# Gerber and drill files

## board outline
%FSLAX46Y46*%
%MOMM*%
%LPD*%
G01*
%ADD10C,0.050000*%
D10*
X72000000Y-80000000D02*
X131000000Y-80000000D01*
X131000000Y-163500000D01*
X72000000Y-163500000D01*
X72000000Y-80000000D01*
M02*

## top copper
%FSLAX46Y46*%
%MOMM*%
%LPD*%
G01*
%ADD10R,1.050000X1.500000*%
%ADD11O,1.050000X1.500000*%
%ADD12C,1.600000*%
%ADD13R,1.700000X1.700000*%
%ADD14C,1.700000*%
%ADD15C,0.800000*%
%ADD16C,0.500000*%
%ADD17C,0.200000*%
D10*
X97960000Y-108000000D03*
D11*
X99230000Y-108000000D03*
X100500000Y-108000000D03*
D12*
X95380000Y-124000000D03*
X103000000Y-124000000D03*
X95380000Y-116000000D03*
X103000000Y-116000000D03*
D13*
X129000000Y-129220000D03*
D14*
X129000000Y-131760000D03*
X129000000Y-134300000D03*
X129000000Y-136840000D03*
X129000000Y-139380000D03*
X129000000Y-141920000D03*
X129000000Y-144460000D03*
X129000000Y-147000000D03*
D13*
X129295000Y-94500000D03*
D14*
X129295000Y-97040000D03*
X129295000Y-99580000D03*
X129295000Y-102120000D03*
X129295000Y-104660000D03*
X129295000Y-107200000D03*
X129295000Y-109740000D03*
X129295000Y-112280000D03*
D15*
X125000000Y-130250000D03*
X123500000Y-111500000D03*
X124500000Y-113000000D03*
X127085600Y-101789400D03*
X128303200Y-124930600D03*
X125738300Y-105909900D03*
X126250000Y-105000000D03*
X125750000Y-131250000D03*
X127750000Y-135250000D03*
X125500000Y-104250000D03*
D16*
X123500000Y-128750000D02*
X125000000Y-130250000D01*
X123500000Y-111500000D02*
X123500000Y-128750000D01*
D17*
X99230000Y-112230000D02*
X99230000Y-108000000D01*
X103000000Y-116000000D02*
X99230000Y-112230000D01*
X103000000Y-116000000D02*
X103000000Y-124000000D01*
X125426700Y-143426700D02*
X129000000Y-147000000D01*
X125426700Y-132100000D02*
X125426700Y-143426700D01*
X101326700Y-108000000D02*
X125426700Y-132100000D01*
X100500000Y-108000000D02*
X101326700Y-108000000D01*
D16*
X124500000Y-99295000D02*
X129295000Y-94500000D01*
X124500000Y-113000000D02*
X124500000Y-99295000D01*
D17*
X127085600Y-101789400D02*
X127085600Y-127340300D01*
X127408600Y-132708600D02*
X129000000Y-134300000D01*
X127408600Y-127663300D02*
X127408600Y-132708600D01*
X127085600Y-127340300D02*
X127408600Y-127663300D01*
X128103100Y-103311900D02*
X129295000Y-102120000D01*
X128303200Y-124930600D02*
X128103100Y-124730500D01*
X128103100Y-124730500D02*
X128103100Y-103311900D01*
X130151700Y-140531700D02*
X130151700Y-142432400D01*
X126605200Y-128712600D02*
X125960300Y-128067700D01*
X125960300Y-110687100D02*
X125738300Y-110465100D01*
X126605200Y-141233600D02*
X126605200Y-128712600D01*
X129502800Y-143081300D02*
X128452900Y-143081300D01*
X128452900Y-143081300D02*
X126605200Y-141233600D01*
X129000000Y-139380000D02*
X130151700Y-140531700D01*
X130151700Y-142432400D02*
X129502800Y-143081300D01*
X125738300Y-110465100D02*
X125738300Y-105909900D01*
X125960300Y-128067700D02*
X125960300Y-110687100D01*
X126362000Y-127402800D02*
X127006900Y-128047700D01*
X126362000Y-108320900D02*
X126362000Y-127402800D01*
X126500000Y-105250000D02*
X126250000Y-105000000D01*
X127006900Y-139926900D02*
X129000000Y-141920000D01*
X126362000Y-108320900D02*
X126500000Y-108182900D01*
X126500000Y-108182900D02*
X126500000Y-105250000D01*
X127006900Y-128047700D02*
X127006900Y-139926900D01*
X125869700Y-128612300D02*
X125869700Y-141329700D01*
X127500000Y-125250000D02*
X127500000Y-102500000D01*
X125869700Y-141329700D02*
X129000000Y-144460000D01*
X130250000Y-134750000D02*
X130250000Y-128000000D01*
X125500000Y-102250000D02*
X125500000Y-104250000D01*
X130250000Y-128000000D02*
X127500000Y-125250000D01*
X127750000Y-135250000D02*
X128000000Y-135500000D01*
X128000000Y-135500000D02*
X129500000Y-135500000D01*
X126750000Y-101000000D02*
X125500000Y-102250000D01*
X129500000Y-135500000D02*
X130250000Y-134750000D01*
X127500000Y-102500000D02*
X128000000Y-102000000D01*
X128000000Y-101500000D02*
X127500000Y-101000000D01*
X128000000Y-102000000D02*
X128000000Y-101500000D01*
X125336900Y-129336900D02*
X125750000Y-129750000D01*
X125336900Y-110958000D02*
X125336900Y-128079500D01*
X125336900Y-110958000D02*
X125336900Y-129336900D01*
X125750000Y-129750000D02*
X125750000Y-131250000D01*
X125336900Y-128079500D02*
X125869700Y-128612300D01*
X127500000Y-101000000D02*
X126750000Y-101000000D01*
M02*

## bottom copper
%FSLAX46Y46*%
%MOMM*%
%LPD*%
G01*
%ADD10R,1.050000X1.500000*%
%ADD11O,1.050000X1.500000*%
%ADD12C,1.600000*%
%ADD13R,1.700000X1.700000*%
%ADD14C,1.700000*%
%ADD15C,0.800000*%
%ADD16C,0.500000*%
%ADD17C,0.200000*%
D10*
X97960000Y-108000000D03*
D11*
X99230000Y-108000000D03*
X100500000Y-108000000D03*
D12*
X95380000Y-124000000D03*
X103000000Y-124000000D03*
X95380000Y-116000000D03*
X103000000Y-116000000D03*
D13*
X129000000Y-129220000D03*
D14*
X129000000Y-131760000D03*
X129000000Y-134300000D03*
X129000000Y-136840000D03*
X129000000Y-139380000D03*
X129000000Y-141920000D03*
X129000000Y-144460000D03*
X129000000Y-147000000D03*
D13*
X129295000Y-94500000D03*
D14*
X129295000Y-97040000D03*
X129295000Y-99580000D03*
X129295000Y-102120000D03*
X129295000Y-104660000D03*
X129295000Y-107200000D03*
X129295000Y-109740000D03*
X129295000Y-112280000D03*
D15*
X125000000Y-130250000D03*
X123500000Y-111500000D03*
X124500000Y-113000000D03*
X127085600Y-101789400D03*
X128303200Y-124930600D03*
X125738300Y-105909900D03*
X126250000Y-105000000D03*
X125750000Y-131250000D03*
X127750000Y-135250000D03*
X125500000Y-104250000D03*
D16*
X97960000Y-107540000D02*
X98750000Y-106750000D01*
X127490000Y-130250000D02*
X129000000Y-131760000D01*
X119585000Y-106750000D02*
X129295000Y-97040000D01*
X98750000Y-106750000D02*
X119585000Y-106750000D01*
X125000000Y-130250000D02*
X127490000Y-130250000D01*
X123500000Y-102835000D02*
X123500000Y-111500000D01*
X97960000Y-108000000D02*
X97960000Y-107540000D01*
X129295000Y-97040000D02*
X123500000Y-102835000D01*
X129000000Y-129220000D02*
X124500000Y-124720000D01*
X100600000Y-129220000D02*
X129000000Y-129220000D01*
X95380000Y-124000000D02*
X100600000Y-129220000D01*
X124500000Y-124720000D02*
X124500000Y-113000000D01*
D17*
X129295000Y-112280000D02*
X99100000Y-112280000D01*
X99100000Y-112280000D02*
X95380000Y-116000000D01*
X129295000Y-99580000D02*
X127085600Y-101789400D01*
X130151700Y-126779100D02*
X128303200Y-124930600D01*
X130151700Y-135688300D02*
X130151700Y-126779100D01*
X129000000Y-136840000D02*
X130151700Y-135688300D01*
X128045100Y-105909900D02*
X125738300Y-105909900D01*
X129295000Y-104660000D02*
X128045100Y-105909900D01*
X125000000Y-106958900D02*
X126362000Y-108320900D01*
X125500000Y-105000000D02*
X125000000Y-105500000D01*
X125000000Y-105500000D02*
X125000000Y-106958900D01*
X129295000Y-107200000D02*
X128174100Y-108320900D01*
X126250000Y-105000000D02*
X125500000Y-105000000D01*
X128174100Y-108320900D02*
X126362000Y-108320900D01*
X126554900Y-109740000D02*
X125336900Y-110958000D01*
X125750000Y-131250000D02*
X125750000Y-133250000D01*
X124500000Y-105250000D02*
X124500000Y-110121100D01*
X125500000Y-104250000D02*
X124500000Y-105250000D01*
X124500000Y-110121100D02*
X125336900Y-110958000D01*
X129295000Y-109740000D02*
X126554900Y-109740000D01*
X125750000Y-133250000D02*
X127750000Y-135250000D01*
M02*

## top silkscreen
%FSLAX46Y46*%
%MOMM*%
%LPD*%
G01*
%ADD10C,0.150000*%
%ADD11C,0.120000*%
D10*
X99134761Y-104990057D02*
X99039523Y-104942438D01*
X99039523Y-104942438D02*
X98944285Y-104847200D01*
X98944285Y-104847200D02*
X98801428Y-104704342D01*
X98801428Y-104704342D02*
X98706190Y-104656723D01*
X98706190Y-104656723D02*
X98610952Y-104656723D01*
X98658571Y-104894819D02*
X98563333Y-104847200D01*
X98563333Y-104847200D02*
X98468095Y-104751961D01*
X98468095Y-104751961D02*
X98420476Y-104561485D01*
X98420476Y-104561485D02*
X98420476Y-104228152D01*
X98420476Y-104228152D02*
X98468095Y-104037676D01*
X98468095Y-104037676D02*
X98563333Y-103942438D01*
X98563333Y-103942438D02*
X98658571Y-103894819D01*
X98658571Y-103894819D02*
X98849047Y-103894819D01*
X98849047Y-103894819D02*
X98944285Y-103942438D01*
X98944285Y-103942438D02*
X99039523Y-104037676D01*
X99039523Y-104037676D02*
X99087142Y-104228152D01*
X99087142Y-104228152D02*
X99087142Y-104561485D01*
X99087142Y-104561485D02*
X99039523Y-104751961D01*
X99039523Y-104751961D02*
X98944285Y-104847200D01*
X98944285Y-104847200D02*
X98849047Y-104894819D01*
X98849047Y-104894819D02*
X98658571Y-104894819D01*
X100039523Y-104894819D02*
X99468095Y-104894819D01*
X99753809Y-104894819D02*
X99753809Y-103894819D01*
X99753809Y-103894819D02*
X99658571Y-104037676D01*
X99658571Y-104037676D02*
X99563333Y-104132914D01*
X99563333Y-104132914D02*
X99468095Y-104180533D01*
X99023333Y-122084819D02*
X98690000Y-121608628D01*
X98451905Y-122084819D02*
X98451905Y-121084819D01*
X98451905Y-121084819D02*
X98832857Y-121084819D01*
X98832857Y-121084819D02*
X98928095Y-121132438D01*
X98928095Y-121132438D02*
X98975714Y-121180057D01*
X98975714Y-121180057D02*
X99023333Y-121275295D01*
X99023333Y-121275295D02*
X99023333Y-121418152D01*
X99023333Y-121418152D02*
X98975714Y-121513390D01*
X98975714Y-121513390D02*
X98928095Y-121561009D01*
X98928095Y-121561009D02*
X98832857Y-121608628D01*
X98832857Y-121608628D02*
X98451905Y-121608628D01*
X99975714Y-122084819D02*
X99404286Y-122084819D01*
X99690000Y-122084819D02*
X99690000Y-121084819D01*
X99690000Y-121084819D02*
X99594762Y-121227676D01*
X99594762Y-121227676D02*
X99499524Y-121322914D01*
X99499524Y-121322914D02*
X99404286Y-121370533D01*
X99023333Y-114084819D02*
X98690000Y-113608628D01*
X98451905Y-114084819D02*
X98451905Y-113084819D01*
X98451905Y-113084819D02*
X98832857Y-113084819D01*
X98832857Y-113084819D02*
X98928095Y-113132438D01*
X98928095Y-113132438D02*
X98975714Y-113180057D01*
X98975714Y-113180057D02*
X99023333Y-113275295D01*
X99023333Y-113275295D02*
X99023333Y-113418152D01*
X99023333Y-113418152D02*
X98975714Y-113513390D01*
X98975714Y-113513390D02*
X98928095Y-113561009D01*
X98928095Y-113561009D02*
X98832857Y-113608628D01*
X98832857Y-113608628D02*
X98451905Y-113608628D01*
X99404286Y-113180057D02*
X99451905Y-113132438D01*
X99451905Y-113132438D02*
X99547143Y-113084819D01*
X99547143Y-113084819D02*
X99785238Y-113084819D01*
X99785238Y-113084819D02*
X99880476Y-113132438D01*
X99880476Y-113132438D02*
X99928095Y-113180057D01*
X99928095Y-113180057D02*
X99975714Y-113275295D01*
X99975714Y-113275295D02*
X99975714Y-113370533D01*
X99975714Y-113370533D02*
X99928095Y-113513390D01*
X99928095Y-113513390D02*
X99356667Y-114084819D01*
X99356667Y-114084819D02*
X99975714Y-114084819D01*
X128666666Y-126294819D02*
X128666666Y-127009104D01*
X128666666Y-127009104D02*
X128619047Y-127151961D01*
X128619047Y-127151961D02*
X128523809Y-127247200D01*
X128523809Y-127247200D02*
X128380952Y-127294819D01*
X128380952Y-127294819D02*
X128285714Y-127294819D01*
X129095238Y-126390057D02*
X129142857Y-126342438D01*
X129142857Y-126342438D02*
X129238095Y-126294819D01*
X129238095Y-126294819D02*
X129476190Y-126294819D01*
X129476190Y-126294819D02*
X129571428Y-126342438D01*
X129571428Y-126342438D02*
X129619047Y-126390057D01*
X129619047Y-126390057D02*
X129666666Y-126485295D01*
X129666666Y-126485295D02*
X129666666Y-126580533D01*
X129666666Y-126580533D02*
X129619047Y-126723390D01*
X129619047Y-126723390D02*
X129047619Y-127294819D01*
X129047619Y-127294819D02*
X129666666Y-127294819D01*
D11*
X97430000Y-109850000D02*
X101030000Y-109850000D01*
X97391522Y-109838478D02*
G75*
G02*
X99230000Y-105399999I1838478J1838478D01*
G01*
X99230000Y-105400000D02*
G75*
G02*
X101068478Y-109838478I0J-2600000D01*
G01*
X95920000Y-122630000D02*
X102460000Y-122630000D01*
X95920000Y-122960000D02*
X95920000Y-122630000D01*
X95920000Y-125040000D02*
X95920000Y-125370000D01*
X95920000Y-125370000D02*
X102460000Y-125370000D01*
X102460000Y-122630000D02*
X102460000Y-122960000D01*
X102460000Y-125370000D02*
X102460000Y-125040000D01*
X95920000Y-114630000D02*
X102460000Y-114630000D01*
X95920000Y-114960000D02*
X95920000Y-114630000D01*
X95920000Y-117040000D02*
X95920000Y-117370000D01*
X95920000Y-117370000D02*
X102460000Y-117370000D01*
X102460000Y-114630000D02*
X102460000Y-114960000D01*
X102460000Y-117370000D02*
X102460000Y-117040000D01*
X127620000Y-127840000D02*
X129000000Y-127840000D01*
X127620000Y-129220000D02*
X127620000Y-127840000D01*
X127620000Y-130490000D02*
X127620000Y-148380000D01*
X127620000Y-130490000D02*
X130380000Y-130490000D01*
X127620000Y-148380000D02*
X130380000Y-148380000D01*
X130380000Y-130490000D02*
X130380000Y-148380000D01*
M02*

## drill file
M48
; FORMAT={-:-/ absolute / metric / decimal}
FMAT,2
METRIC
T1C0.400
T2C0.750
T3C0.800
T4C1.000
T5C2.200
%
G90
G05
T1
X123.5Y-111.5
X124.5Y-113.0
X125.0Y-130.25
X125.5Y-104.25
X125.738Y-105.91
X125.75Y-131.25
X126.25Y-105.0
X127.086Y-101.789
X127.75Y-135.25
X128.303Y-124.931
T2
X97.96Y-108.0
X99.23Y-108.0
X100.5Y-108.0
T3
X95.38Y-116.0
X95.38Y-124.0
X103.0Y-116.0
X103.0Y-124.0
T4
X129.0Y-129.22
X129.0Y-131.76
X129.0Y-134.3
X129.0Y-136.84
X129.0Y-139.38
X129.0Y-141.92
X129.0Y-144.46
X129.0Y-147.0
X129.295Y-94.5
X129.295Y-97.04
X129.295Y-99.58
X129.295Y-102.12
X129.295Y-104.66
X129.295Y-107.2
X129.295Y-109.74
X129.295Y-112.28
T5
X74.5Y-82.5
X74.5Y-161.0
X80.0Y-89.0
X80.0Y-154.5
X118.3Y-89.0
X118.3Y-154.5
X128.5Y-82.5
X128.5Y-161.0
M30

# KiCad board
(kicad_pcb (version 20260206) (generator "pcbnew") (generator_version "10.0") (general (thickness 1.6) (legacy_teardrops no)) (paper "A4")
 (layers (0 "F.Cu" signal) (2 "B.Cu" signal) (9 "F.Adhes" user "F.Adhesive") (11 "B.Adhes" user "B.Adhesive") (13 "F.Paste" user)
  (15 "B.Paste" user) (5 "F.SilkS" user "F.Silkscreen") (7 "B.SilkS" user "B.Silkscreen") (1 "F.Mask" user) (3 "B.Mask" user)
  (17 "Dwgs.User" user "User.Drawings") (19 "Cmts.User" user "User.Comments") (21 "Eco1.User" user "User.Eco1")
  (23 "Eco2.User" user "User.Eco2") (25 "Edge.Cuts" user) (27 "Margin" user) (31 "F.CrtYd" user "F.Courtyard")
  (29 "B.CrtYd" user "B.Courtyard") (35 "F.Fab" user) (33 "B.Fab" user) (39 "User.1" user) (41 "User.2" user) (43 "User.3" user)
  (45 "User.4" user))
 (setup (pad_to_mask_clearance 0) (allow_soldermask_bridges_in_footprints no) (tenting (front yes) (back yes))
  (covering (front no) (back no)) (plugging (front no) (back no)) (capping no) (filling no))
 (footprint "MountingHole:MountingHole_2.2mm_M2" (layer "F.Cu") (at 118.3 89)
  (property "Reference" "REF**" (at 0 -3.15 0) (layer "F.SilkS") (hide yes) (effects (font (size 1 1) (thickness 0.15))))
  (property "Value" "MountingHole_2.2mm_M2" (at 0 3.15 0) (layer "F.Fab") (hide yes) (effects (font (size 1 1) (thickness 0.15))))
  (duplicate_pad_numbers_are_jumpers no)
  (pad "" np_thru_hole circle (at 0 0) (size 2.2 2.2) (drill 2.2) (layers "*.Cu" "*.Mask")))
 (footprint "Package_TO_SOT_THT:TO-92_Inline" (layer "F.Cu") (at 97.96 108)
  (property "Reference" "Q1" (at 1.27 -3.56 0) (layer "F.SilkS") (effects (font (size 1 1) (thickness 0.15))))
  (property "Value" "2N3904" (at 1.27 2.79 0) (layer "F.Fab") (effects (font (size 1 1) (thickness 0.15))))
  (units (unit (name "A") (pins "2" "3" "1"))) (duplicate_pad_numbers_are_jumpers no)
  (fp_line (start -0.53 1.85) (end 3.07 1.85) (stroke (width 0.12) (type solid)) (layer "F.SilkS"))
  (fp_arc (start -0.568478 1.838478) (mid -1.132087 -0.994977) (end 1.27 -2.6) (stroke (width 0.12) (type solid)) (layer "F.SilkS"))
  (fp_arc (start 1.27 -2.6) (mid 3.672087 -0.994977) (end 3.108478 1.838478) (stroke (width 0.12) (type solid)) (layer "F.SilkS"))
  (pad "1" thru_hole rect (at 0 0) (size 1.05 1.5) (drill 0.75) (layers "*.Cu" "*.Mask") (remove_unused_layers no) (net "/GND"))
  (pad "2" thru_hole oval (at 1.27 0) (size 1.05 1.5) (drill 0.75) (layers "*.Cu" "*.Mask") (remove_unused_layers no) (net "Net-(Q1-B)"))
  (pad "3" thru_hole oval (at 2.54 0) (size 1.05 1.5) (drill 0.75) (layers "*.Cu" "*.Mask") (remove_unused_layers no) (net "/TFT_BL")))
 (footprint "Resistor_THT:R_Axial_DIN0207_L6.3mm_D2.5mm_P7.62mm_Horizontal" (layer "F.Cu") (at 95.38 124)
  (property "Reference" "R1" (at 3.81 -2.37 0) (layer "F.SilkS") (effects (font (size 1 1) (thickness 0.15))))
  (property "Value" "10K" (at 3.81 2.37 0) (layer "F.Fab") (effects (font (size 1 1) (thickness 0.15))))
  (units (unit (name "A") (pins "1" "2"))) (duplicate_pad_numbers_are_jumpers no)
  (fp_line (start 0.54 -1.37) (end 7.08 -1.37) (stroke (width 0.12) (type solid)) (layer "F.SilkS"))
  (fp_line (start 0.54 -1.04) (end 0.54 -1.37) (stroke (width 0.12) (type solid)) (layer "F.SilkS"))
  (fp_line (start 0.54 1.04) (end 0.54 1.37) (stroke (width 0.12) (type solid)) (layer "F.SilkS"))
  (fp_line (start 0.54 1.37) (end 7.08 1.37) (stroke (width 0.12) (type solid)) (layer "F.SilkS"))
  (fp_line (start 7.08 -1.37) (end 7.08 -1.04) (stroke (width 0.12) (type solid)) (layer "F.SilkS"))
  (fp_line (start 7.08 1.37) (end 7.08 1.04) (stroke (width 0.12) (type solid)) (layer "F.SilkS"))
  (pad "1" thru_hole circle (at 0 0) (size 1.6 1.6) (drill 0.8) (layers "*.Cu" "*.Mask") (remove_unused_layers no) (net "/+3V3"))
  (pad "2" thru_hole circle (at 7.62 0) (size 1.6 1.6) (drill 0.8) (layers "*.Cu" "*.Mask") (remove_unused_layers no) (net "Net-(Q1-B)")))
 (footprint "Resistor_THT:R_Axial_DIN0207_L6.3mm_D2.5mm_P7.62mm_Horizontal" (layer "F.Cu") (at 95.38 116)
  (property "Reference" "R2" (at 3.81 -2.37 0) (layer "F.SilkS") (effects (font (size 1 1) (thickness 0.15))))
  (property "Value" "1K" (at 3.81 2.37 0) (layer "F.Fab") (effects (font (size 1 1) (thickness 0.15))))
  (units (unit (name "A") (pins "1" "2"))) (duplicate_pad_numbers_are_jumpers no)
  (fp_line (start 0.54 -1.37) (end 7.08 -1.37) (stroke (width 0.12) (type solid)) (layer "F.SilkS"))
  (fp_line (start 0.54 -1.04) (end 0.54 -1.37) (stroke (width 0.12) (type solid)) (layer "F.SilkS"))
  (fp_line (start 0.54 1.04) (end 0.54 1.37) (stroke (width 0.12) (type solid)) (layer "F.SilkS"))
  (fp_line (start 0.54 1.37) (end 7.08 1.37) (stroke (width 0.12) (type solid)) (layer "F.SilkS"))
  (fp_line (start 7.08 -1.37) (end 7.08 -1.04) (stroke (width 0.12) (type solid)) (layer "F.SilkS"))
  (fp_line (start 7.08 1.37) (end 7.08 1.04) (stroke (width 0.12) (type solid)) (layer "F.SilkS"))
  (pad "1" thru_hole circle (at 0 0) (size 1.6 1.6) (drill 0.8) (layers "*.Cu" "*.Mask") (remove_unused_layers no) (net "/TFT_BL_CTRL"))
  (pad "2" thru_hole circle (at 7.62 0) (size 1.6 1.6) (drill 0.8) (layers "*.Cu" "*.Mask") (remove_unused_layers no) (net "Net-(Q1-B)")))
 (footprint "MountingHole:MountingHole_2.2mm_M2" (layer "F.Cu") (at 80 154.5)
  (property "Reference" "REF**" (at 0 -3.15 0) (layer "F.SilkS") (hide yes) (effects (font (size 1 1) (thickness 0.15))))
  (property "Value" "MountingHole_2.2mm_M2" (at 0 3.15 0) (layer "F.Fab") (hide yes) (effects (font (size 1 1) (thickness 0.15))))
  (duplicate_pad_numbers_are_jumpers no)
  (pad "" np_thru_hole circle (at 0 0) (size 2.2 2.2) (drill 2.2) (layers "*.Cu" "*.Mask")))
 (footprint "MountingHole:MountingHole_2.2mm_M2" (layer "F.Cu") (at 128.5 161)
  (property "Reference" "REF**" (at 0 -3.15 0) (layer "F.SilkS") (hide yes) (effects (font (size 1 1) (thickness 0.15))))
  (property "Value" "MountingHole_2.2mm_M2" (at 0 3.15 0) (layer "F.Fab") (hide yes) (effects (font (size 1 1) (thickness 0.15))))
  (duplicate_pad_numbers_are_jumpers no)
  (pad "" np_thru_hole circle (at 0 0) (size 2.2 2.2) (drill 2.2) (layers "*.Cu" "*.Mask")))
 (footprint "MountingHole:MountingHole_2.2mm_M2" (layer "F.Cu") (at 128.5 82.5)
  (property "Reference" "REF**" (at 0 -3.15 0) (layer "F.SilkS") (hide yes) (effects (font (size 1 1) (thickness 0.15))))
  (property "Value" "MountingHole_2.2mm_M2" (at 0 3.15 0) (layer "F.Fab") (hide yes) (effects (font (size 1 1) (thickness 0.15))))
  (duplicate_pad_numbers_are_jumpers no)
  (pad "" np_thru_hole circle (at 0 0) (size 2.2 2.2) (drill 2.2) (layers "*.Cu" "*.Mask")))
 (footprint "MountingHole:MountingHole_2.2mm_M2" (layer "F.Cu") (at 80 89)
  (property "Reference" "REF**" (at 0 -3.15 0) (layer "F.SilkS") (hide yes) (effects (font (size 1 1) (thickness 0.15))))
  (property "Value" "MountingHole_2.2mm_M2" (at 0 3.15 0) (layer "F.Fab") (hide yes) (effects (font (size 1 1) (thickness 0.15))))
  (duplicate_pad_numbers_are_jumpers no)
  (pad "" np_thru_hole circle (at 0 0) (size 2.2 2.2) (drill 2.2) (layers "*.Cu" "*.Mask")))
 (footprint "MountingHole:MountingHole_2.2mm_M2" (layer "F.Cu") (at 118.3 154.5)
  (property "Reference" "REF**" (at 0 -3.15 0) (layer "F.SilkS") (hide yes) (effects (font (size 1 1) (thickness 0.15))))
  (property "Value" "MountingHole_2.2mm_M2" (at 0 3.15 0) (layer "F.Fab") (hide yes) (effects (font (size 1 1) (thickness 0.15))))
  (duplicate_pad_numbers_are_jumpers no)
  (pad "" np_thru_hole circle (at 0 0) (size 2.2 2.2) (drill 2.2) (layers "*.Cu" "*.Mask")))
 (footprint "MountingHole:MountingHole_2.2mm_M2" (layer "F.Cu") (at 74.5 82.5)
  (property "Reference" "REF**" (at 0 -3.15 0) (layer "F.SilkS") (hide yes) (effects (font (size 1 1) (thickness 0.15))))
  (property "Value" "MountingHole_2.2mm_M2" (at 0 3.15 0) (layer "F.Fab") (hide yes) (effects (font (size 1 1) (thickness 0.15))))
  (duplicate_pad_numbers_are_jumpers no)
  (pad "" np_thru_hole circle (at 0 0) (size 2.2 2.2) (drill 2.2) (layers "*.Cu" "*.Mask")))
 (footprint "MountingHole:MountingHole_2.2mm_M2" (layer "F.Cu") (at 74.5 161)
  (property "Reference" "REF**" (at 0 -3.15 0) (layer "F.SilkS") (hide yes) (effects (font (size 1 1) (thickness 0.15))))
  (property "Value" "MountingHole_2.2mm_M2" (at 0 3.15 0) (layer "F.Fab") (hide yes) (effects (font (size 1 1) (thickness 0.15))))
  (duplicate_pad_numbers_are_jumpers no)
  (pad "" np_thru_hole circle (at 0 0) (size 2.2 2.2) (drill 2.2) (layers "*.Cu" "*.Mask")))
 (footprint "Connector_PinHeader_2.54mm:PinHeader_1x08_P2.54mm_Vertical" (layer "F.Cu") (at 129 129.22)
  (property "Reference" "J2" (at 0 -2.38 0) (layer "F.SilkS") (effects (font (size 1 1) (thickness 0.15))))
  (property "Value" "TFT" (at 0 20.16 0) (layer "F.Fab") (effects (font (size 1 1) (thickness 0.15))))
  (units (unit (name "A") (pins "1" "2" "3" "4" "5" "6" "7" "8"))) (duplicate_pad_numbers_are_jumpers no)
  (fp_line (start -1.38 -1.38) (end 0 -1.38) (stroke (width 0.12) (type solid)) (layer "F.SilkS"))
  (fp_line (start -1.38 0) (end -1.38 -1.38) (stroke (width 0.12) (type solid)) (layer "F.SilkS"))
  (fp_line (start -1.38 1.27) (end -1.38 19.16) (stroke (width 0.12) (type solid)) (layer "F.SilkS"))
  (fp_line (start -1.38 1.27) (end 1.38 1.27) (stroke (width 0.12) (type solid)) (layer "F.SilkS"))
  (fp_line (start -1.38 19.16) (end 1.38 19.16) (stroke (width 0.12) (type solid)) (layer "F.SilkS"))
  (fp_line (start 1.38 1.27) (end 1.38 19.16) (stroke (width 0.12) (type solid)) (layer "F.SilkS"))
  (pad "1" thru_hole rect (at 0 0) (size 1.7 1.7) (drill 1) (layers "*.Cu" "*.Mask") (remove_unused_layers no) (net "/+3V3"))
  (pad "2" thru_hole circle (at 0 2.54) (size 1.7 1.7) (drill 1) (layers "*.Cu" "*.Mask") (remove_unused_layers no) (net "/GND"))
  (pad "3" thru_hole circle (at 0 5.08) (size 1.7 1.7) (drill 1) (layers "*.Cu" "*.Mask") (remove_unused_layers no) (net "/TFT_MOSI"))
  (pad "4" thru_hole circle (at 0 7.62) (size 1.7 1.7) (drill 1) (layers "*.Cu" "*.Mask") (remove_unused_layers no) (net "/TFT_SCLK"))
  (pad "5" thru_hole circle (at 0 10.16) (size 1.7 1.7) (drill 1) (layers "*.Cu" "*.Mask") (remove_unused_layers no) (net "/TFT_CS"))
  (pad "6" thru_hole circle (at 0 12.7) (size 1.7 1.7) (drill 1) (layers "*.Cu" "*.Mask") (remove_unused_layers no) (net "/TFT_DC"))
  (pad "7" thru_hole circle (at 0 15.24) (size 1.7 1.7) (drill 1) (layers "*.Cu" "*.Mask") (remove_unused_layers no) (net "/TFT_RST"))
  (pad "8" thru_hole circle (at 0 17.78) (size 1.7 1.7) (drill 1) (layers "*.Cu" "*.Mask") (remove_unused_layers no) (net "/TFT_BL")))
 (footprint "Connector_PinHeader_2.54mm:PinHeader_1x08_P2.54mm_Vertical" (layer "B.Cu") (at 129.295 94.5 180)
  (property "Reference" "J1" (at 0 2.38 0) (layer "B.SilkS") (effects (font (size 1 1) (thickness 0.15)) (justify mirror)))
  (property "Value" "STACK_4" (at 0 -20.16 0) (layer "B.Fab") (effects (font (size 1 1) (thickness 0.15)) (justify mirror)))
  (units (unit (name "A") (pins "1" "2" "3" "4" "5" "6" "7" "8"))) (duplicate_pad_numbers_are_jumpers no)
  (pad "1" thru_hole rect (at 0 0 180) (size 1.7 1.7) (drill 1) (layers "*.Cu" "*.Mask") (remove_unused_layers no) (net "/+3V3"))
  (pad "2" thru_hole circle (at 0 -2.54 180) (size 1.7 1.7) (drill 1) (layers "*.Cu" "*.Mask") (remove_unused_layers no) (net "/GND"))
  (pad "3" thru_hole circle (at 0 -5.08 180) (size 1.7 1.7) (drill 1) (layers "*.Cu" "*.Mask") (remove_unused_layers no) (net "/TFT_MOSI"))
  (pad "4" thru_hole circle (at 0 -7.62 180) (size 1.7 1.7) (drill 1) (layers "*.Cu" "*.Mask") (remove_unused_layers no) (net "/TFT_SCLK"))
  (pad "5" thru_hole circle (at 0 -10.16 180) (size 1.7 1.7) (drill 1) (layers "*.Cu" "*.Mask") (remove_unused_layers no) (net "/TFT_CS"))
  (pad "6" thru_hole circle (at 0 -12.7 180) (size 1.7 1.7) (drill 1) (layers "*.Cu" "*.Mask") (remove_unused_layers no) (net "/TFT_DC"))
  (pad "7" thru_hole circle (at 0 -15.24 180) (size 1.7 1.7) (drill 1) (layers "*.Cu" "*.Mask") (remove_unused_layers no) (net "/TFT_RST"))
  (pad "8" thru_hole circle (at 0 -17.78 180) (size 1.7 1.7) (drill 1) (layers "*.Cu" "*.Mask") (remove_unused_layers no)
   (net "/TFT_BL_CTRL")))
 (gr_rect (start 72 80) (end 131 163.5) (stroke (width 0.05) (type default)) (fill no) (layer "Edge.Cuts"))
 (segment (start 123.5 128.75) (end 125 130.25) (width 0.5) (layer "F.Cu") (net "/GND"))
 (segment (start 123.5 111.5) (end 123.5 128.75) (width 0.5) (layer "F.Cu") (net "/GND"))
 (via (at 125 130.25) (size 0.8) (drill 0.4) (layers "F.Cu" "B.Cu") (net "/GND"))
 (via (at 123.5 111.5) (size 0.8) (drill 0.4) (layers "F.Cu" "B.Cu") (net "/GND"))
 (segment (start 97.96 107.54) (end 98.75 106.75) (width 0.5) (layer "B.Cu") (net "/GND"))
 (segment (start 127.49 130.25) (end 129 131.76) (width 0.5) (layer "B.Cu") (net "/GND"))
 (segment (start 119.585 106.75) (end 129.295 97.04) (width 0.5) (layer "B.Cu") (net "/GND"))
 (segment (start 98.75 106.75) (end 119.585 106.75) (width 0.5) (layer "B.Cu") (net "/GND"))
 (segment (start 125 130.25) (end 127.49 130.25) (width 0.5) (layer "B.Cu") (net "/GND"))
 (segment (start 123.5 102.835) (end 123.5 111.5) (width 0.5) (layer "B.Cu") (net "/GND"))
 (segment (start 97.96 108) (end 97.96 107.54) (width 0.5) (layer "B.Cu") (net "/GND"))
 (segment (start 129.295 97.04) (end 123.5 102.835) (width 0.5) (layer "B.Cu") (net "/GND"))
 (segment (start 99.23 112.23) (end 99.23 108) (width 0.2) (layer "F.Cu") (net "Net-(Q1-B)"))
 (segment (start 103 116) (end 99.23 112.23) (width 0.2) (layer "F.Cu") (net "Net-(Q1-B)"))
 (segment (start 103 116) (end 103 124) (width 0.2) (layer "F.Cu") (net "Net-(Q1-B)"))
 (segment (start 125.4267 143.4267) (end 129 147) (width 0.2) (layer "F.Cu") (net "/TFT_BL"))
 (segment (start 125.4267 132.1) (end 125.4267 143.4267) (width 0.2) (layer "F.Cu") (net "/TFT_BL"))
 (segment (start 101.3267 108) (end 125.4267 132.1) (width 0.2) (layer "F.Cu") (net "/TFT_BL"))
 (segment (start 100.5 108) (end 101.3267 108) (width 0.2) (layer "F.Cu") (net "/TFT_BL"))
 (segment (start 124.5 99.295) (end 129.295 94.5) (width 0.5) (layer "F.Cu") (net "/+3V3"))
 (segment (start 124.5 113) (end 124.5 99.295) (width 0.5) (layer "F.Cu") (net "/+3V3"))
 (via (at 124.5 113) (size 0.8) (drill 0.4) (layers "F.Cu" "B.Cu") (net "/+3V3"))
 (segment (start 129 129.22) (end 124.5 124.72) (width 0.5) (layer "B.Cu") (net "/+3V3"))
 (segment (start 100.6 129.22) (end 129 129.22) (width 0.5) (layer "B.Cu") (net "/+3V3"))
 (segment (start 95.38 124) (end 100.6 129.22) (width 0.5) (layer "B.Cu") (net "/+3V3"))
 (segment (start 124.5 124.72) (end 124.5 113) (width 0.5) (layer "B.Cu") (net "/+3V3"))
 (segment (start 129.295 112.28) (end 99.1 112.28) (width 0.2) (layer "B.Cu") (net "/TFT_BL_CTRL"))
 (segment (start 99.1 112.28) (end 95.38 116) (width 0.2) (layer "B.Cu") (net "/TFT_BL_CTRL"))
 (segment (start 127.0856 101.7894) (end 127.0856 127.3403) (width 0.2) (layer "F.Cu") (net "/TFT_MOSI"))
 (segment (start 127.4086 132.7086) (end 129 134.3) (width 0.2) (layer "F.Cu") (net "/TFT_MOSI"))
 (segment (start 127.4086 127.6633) (end 127.4086 132.7086) (width 0.2) (layer "F.Cu") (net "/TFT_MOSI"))
 (segment (start 127.0856 127.3403) (end 127.4086 127.6633) (width 0.2) (layer "F.Cu") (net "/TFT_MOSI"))
 (via (at 127.0856 101.7894) (size 0.8) (drill 0.4) (layers "F.Cu" "B.Cu") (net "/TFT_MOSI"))
 (segment (start 129.295 99.58) (end 127.0856 101.7894) (width 0.2) (layer "B.Cu") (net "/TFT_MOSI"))
 (segment (start 128.1031 103.3119) (end 129.295 102.12) (width 0.2) (layer "F.Cu") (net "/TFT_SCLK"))
 (segment (start 128.3032 124.9306) (end 128.1031 124.7305) (width 0.2) (layer "F.Cu") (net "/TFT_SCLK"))
 (segment (start 128.1031 124.7305) (end 128.1031 103.3119) (width 0.2) (layer "F.Cu") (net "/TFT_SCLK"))
 (via (at 128.3032 124.9306) (size 0.8) (drill 0.4) (layers "F.Cu" "B.Cu") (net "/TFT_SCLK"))
 (segment (start 130.1517 126.7791) (end 128.3032 124.9306) (width 0.2) (layer "B.Cu") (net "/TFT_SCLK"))
 (segment (start 130.1517 135.6883) (end 130.1517 126.7791) (width 0.2) (layer "B.Cu") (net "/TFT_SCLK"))
 (segment (start 129 136.84) (end 130.1517 135.6883) (width 0.2) (layer "B.Cu") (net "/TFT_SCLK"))
 (segment (start 130.1517 140.5317) (end 130.1517 142.4324) (width 0.2) (layer "F.Cu") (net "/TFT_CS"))
 (segment (start 126.6052 128.7126) (end 125.9603 128.0677) (width 0.2) (layer "F.Cu") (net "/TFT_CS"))
 (segment (start 125.9603 110.6871) (end 125.7383 110.4651) (width 0.2) (layer "F.Cu") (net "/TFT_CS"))
 (segment (start 126.6052 141.2336) (end 126.6052 128.7126) (width 0.2) (layer "F.Cu") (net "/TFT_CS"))
 (segment (start 129.5028 143.0813) (end 128.4529 143.0813) (width 0.2) (layer "F.Cu") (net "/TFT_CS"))
 (segment (start 128.4529 143.0813) (end 126.6052 141.2336) (width 0.2) (layer "F.Cu") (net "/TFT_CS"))
 (segment (start 129 139.38) (end 130.1517 140.5317) (width 0.2) (layer "F.Cu") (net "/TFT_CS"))
 (segment (start 130.1517 142.4324) (end 129.5028 143.0813) (width 0.2) (layer "F.Cu") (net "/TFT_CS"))
 (segment (start 125.7383 110.4651) (end 125.7383 105.9099) (width 0.2) (layer "F.Cu") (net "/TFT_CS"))
 (segment (start 125.9603 128.0677) (end 125.9603 110.6871) (width 0.2) (layer "F.Cu") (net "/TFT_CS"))
 (via (at 125.7383 105.9099) (size 0.8) (drill 0.4) (layers "F.Cu" "B.Cu") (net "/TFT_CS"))
 (segment (start 128.0451 105.9099) (end 125.7383 105.9099) (width 0.2) (layer "B.Cu") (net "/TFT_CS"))
 (segment (start 129.295 104.66) (end 128.0451 105.9099) (width 0.2) (layer "B.Cu") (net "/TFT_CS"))
 (segment (start 126.362 127.4028) (end 127.0069 128.0477) (width 0.2) (layer "F.Cu") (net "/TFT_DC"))
 (segment (start 126.362 108.3209) (end 126.362 127.4028) (width 0.2) (layer "F.Cu") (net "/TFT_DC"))
 (segment (start 126.5 105.25) (end 126.25 105) (width 0.2) (layer "F.Cu") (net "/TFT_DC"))
 (segment (start 127.0069 139.9269) (end 129 141.92) (width 0.2) (layer "F.Cu") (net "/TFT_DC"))
 (segment (start 126.362 108.3209) (end 126.5 108.1829) (width 0.2) (layer "F.Cu") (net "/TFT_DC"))
 (segment (start 126.5 108.1829) (end 126.5 105.25) (width 0.2) (layer "F.Cu") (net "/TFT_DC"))
 (segment (start 127.0069 128.0477) (end 127.0069 139.9269) (width 0.2) (layer "F.Cu") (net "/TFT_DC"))
 (via (at 126.25 105) (size 0.8) (drill 0.4) (layers "F.Cu" "B.Cu") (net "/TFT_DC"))
 (segment (start 125 106.9589) (end 126.362 108.3209) (width 0.2) (layer "B.Cu") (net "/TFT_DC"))
 (segment (start 125.5 105) (end 125 105.5) (width 0.2) (layer "B.Cu") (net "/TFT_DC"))
 (segment (start 125 105.5) (end 125 106.9589) (width 0.2) (layer "B.Cu") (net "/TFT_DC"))
 (segment (start 129.295 107.2) (end 128.1741 108.3209) (width 0.2) (layer "B.Cu") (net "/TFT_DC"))
 (segment (start 126.25 105) (end 125.5 105) (width 0.2) (layer "B.Cu") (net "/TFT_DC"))
 (segment (start 128.1741 108.3209) (end 126.362 108.3209) (width 0.2) (layer "B.Cu") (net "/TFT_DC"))
 (segment (start 125.8697 128.6123) (end 125.8697 141.3297) (width 0.2) (layer "F.Cu") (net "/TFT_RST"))
 (segment (start 127.5 125.25) (end 127.5 102.5) (width 0.2) (layer "F.Cu") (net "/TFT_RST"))
 (segment (start 125.8697 141.3297) (end 129 144.46) (width 0.2) (layer "F.Cu") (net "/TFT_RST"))
 (segment (start 130.25 134.75) (end 130.25 128) (width 0.2) (layer "F.Cu") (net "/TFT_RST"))
 (segment (start 125.5 102.25) (end 125.5 104.25) (width 0.2) (layer "F.Cu") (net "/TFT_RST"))
 (segment (start 130.25 128) (end 127.5 125.25) (width 0.2) (layer "F.Cu") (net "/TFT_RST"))
 (segment (start 127.75 135.25) (end 128 135.5) (width 0.2) (layer "F.Cu") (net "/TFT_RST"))
 (segment (start 128 135.5) (end 129.5 135.5) (width 0.2) (layer "F.Cu") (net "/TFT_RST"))
 (segment (start 126.75 101) (end 125.5 102.25) (width 0.2) (layer "F.Cu") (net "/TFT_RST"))
 (segment (start 129.5 135.5) (end 130.25 134.75) (width 0.2) (layer "F.Cu") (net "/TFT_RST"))
 (segment (start 127.5 102.5) (end 128 102) (width 0.2) (layer "F.Cu") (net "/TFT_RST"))
 (segment (start 128 101.5) (end 127.5 101) (width 0.2) (layer "F.Cu") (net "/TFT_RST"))
 (segment (start 128 102) (end 128 101.5) (width 0.2) (layer "F.Cu") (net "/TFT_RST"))
 (segment (start 125.3369 129.3369) (end 125.75 129.75) (width 0.2) (layer "F.Cu") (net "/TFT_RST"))
 (segment (start 125.3369 110.958) (end 125.3369 128.0795) (width 0.2) (layer "F.Cu") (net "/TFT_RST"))
 (segment (start 125.3369 110.958) (end 125.3369 129.3369) (width 0.2) (layer "F.Cu") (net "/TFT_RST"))
 (segment (start 125.75 129.75) (end 125.75 131.25) (width 0.2) (layer "F.Cu") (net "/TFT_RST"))
 (segment (start 125.3369 128.0795) (end 125.8697 128.6123) (width 0.2) (layer "F.Cu") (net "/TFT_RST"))
 (segment (start 127.5 101) (end 126.75 101) (width 0.2) (layer "F.Cu") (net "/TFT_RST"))
 (via (at 125.75 131.25) (size 0.8) (drill 0.4) (layers "F.Cu" "B.Cu") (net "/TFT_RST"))
 (via (at 127.75 135.25) (size 0.8) (drill 0.4) (layers "F.Cu" "B.Cu") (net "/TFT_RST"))
 (via (at 125.5 104.25) (size 0.8) (drill 0.4) (layers "F.Cu" "B.Cu") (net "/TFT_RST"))
 (segment (start 126.5549 109.74) (end 125.3369 110.958) (width 0.2) (layer "B.Cu") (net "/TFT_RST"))
 (segment (start 125.75 131.25) (end 125.75 133.25) (width 0.2) (layer "B.Cu") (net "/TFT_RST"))
 (segment (start 124.5 105.25) (end 124.5 110.1211) (width 0.2) (layer "B.Cu") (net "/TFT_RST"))
 (segment (start 125.5 104.25) (end 124.5 105.25) (width 0.2) (layer "B.Cu") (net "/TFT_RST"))
 (segment (start 124.5 110.1211) (end 125.3369 110.958) (width 0.2) (layer "B.Cu") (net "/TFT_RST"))
 (segment (start 129.295 109.74) (end 126.5549 109.74) (width 0.2) (layer "B.Cu") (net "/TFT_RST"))
 (segment (start 125.75 133.25) (end 127.75 135.25) (width 0.2) (layer "B.Cu") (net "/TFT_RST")))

